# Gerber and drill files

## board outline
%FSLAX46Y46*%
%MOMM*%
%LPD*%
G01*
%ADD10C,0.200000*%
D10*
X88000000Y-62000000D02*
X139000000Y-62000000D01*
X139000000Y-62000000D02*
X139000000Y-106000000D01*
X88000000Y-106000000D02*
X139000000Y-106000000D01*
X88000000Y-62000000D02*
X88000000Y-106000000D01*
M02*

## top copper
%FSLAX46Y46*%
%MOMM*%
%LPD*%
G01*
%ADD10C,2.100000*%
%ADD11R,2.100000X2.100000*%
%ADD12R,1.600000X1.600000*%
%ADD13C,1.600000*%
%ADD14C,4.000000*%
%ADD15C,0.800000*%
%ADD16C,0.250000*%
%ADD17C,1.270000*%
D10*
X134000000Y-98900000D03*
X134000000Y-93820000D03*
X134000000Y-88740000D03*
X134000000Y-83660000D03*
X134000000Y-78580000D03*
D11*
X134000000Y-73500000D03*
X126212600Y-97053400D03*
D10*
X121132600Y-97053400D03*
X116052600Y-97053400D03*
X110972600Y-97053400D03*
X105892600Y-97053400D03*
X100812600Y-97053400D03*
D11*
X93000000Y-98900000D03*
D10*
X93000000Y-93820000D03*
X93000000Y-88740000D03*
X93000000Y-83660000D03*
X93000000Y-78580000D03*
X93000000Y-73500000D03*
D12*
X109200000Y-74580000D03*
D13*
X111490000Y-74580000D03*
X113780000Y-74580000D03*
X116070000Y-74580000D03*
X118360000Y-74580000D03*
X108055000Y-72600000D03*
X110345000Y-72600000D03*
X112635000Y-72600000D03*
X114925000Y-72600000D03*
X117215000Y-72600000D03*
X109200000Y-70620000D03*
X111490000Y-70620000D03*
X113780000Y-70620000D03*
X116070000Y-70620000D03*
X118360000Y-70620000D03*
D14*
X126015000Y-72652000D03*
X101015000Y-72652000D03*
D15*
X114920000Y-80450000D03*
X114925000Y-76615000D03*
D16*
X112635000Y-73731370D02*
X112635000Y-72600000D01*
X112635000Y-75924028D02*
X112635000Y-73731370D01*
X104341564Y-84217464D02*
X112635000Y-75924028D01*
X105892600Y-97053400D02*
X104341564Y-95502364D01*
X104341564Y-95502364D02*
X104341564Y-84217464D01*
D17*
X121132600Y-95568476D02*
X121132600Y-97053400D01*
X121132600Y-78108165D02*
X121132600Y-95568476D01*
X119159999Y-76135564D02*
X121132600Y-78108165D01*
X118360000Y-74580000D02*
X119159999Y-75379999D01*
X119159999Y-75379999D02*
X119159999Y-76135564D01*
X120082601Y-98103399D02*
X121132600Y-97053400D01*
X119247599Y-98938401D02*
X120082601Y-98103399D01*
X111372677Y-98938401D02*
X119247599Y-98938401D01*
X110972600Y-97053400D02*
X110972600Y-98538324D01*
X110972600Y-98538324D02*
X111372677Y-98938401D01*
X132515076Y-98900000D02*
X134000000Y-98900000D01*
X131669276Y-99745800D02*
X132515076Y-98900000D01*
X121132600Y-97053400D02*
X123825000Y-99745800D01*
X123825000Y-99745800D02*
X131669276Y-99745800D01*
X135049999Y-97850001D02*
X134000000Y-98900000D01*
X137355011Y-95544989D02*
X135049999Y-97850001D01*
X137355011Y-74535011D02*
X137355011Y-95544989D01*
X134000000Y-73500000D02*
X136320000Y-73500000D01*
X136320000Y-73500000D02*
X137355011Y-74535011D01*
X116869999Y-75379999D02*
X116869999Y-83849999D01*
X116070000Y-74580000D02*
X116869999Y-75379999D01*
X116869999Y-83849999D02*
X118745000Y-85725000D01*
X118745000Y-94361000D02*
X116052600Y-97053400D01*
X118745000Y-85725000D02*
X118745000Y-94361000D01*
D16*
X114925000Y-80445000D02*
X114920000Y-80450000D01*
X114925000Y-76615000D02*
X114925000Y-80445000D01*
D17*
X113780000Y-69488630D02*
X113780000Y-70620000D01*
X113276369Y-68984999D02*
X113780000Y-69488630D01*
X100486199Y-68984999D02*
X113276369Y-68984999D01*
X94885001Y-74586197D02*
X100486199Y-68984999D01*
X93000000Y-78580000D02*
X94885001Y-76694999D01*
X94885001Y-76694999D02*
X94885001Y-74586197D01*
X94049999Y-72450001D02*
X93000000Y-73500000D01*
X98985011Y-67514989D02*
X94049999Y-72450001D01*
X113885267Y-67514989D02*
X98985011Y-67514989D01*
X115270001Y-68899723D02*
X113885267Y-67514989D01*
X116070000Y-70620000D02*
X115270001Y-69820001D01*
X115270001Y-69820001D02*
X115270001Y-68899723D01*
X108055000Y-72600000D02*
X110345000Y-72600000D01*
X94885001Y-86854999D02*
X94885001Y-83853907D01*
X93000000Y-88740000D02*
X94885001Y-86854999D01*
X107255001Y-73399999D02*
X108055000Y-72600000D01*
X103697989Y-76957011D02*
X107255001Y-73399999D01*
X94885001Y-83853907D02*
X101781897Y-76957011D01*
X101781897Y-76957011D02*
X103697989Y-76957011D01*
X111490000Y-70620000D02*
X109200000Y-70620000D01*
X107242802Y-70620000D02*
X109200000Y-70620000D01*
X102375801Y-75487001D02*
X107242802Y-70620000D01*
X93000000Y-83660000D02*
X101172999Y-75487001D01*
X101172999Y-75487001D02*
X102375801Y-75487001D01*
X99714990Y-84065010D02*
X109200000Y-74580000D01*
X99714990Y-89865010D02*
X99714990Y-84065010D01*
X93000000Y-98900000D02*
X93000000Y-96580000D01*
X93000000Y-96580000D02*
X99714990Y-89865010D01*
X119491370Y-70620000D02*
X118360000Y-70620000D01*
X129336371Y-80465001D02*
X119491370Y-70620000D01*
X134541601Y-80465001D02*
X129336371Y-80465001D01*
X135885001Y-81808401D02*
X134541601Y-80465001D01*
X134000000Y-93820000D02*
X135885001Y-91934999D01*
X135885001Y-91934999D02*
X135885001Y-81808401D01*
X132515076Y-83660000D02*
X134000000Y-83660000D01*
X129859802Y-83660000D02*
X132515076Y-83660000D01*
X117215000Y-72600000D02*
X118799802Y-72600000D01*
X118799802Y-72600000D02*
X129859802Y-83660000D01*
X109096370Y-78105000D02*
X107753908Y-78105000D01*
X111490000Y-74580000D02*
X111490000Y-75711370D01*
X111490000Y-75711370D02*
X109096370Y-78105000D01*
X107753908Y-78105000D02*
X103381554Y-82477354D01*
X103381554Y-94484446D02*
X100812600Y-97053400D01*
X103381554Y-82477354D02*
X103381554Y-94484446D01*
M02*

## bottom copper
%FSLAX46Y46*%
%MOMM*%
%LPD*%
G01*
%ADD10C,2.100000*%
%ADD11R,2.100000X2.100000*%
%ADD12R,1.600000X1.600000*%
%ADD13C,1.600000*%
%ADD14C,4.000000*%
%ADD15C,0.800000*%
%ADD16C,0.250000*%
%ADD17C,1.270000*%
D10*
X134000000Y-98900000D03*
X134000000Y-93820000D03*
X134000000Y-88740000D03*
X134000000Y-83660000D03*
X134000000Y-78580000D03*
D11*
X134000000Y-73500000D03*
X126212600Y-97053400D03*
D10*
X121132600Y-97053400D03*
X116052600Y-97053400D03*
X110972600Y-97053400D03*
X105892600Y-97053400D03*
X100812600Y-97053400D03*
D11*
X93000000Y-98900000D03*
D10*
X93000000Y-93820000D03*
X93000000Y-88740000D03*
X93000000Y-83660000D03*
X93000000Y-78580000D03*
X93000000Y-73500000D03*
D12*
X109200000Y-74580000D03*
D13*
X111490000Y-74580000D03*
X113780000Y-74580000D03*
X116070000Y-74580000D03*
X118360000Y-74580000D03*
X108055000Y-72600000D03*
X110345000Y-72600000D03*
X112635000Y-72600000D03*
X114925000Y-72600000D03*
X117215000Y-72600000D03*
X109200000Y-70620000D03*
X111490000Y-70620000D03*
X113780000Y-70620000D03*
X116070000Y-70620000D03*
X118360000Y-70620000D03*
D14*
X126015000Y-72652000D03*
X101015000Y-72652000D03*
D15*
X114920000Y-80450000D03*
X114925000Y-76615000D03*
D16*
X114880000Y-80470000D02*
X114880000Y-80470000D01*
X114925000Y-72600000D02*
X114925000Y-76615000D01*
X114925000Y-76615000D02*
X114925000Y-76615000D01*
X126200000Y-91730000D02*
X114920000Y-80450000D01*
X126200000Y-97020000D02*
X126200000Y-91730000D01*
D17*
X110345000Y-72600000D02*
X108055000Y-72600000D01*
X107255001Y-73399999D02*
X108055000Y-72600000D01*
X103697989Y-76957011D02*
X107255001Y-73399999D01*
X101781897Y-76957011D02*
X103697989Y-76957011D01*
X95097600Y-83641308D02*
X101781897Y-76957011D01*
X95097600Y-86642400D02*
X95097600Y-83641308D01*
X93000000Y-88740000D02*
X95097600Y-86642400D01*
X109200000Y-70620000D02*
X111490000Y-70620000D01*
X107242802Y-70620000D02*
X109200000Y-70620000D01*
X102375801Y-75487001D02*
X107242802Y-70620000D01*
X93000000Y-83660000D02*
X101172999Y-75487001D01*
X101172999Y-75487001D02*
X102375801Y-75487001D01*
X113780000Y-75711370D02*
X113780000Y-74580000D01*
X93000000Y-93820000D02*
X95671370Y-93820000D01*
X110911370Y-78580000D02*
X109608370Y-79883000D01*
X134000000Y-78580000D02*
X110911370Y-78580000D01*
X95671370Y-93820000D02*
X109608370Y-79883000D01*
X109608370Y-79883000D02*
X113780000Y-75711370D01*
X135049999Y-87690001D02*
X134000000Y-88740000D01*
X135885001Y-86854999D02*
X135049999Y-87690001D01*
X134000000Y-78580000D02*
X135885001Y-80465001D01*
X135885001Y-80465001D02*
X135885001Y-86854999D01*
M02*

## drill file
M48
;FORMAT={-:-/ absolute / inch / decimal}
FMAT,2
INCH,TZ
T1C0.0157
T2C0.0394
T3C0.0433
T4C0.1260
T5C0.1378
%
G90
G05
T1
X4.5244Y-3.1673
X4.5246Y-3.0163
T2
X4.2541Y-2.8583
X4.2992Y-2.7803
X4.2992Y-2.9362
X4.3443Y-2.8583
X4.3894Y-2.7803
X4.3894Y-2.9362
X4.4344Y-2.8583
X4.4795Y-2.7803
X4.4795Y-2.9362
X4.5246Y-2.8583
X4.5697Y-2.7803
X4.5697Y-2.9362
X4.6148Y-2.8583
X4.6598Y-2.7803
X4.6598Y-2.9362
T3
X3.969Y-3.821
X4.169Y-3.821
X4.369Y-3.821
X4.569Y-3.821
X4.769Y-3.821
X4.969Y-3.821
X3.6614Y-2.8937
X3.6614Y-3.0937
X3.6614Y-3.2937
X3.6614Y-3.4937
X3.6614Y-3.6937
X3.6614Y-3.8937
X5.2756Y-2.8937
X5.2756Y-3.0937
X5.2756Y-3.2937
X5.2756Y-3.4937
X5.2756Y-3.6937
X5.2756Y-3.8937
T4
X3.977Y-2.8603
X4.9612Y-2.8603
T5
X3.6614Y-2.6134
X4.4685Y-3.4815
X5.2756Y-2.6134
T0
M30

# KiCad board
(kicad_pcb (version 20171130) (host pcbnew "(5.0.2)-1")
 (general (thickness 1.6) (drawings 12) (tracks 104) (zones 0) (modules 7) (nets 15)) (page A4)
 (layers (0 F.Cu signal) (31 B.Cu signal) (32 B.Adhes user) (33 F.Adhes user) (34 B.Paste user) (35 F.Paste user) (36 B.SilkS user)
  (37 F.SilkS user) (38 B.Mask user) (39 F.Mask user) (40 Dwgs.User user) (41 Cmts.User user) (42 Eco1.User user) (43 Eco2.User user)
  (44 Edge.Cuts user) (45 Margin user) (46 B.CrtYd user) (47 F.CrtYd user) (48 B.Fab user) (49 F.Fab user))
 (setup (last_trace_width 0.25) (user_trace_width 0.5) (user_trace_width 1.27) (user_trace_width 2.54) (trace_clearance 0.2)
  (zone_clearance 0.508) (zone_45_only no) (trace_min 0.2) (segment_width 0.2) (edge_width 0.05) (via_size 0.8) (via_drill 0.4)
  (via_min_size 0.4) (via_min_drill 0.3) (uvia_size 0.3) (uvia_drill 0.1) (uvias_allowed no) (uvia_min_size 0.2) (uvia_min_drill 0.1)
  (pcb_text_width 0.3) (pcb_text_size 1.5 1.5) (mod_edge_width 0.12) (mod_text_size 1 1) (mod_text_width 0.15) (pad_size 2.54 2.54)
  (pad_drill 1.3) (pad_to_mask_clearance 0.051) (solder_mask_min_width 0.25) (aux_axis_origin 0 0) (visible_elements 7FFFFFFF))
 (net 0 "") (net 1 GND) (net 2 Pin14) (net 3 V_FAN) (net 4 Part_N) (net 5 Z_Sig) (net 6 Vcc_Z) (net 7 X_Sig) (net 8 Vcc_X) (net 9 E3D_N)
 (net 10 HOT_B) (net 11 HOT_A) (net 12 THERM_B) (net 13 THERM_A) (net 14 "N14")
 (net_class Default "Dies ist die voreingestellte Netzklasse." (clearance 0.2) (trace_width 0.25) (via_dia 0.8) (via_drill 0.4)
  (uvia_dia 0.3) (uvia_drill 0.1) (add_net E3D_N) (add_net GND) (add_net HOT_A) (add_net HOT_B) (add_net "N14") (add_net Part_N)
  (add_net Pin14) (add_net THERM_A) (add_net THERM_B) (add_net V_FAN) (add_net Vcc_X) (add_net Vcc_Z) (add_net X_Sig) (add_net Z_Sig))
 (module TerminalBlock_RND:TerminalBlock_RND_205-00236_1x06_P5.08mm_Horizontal (layer F.Cu) (at 134 73.5 270)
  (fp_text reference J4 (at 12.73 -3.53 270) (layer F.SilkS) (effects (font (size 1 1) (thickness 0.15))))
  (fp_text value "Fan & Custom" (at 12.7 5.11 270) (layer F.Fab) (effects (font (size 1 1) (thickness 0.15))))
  (pad 6 thru_hole circle (at 25.4 0 270) (size 2.1 2.1) (drill 1.1) (layers *.Cu *.Mask) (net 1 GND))
  (pad 5 thru_hole circle (at 20.32 0 270) (size 2.1 2.1) (drill 1.1) (layers *.Cu *.Mask) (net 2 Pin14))
  (pad 4 thru_hole circle (at 15.24 0 270) (size 2.1 2.1) (drill 1.1) (layers *.Cu *.Mask) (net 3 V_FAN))
  (pad 3 thru_hole circle (at 10.16 0 270) (size 2.1 2.1) (drill 1.1) (layers *.Cu *.Mask) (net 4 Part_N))
  (pad 2 thru_hole circle (at 5.08 0 270) (size 2.1 2.1) (drill 1.1) (layers *.Cu *.Mask) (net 3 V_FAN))
  (pad 1 thru_hole rect (at 0 0 270) (size 2.1 2.1) (drill 1.1) (layers *.Cu *.Mask) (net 1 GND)))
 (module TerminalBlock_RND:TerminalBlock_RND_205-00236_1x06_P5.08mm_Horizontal (layer F.Cu) (at 126.2126 97.0534 180)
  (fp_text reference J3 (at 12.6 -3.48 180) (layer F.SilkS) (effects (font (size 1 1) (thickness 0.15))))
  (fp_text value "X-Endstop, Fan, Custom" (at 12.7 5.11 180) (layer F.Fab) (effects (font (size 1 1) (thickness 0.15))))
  (pad 1 thru_hole rect (at 0 0 180) (size 2.1 2.1) (drill 1.1) (layers *.Cu *.Mask) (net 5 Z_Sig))
  (pad 2 thru_hole circle (at 5.08 0 180) (size 2.1 2.1) (drill 1.1) (layers *.Cu *.Mask) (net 1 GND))
  (pad 3 thru_hole circle (at 10.16 0 180) (size 2.1 2.1) (drill 1.1) (layers *.Cu *.Mask) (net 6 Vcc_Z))
  (pad 4 thru_hole circle (at 15.24 0 180) (size 2.1 2.1) (drill 1.1) (layers *.Cu *.Mask) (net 1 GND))
  (pad 5 thru_hole circle (at 20.32 0 180) (size 2.1 2.1) (drill 1.1) (layers *.Cu *.Mask) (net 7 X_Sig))
  (pad 6 thru_hole circle (at 25.4 0 180) (size 2.1 2.1) (drill 1.1) (layers *.Cu *.Mask) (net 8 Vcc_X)))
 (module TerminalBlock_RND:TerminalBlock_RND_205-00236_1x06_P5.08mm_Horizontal (layer F.Cu) (at 93 98.9 90)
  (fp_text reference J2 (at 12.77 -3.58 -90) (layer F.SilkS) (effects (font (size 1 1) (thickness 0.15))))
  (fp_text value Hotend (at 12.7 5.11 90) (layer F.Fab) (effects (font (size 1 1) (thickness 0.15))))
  (pad 1 thru_hole rect (at 0 0 90) (size 2.1 2.1) (drill 1.1) (layers *.Cu *.Mask) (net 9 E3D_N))
  (pad 2 thru_hole circle (at 5.08 0 90) (size 2.1 2.1) (drill 1.1) (layers *.Cu *.Mask) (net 3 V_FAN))
  (pad 3 thru_hole circle (at 10.16 0 90) (size 2.1 2.1) (drill 1.1) (layers *.Cu *.Mask) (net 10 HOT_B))
  (pad 4 thru_hole circle (at 15.24 0 90) (size 2.1 2.1) (drill 1.1) (layers *.Cu *.Mask) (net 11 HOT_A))
  (pad 5 thru_hole circle (at 20.32 0 90) (size 2.1 2.1) (drill 1.1) (layers *.Cu *.Mask) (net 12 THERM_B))
  (pad 6 thru_hole circle (at 25.4 0 90) (size 2.1 2.1) (drill 1.1) (layers *.Cu *.Mask) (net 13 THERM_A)))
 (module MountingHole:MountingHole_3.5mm (layer F.Cu) (at 113.5 88.43)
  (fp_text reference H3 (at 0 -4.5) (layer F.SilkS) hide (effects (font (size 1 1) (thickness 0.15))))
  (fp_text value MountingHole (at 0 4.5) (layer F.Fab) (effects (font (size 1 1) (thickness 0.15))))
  (pad 1 np_thru_hole circle (at 0 0) (size 3.5 3.5) (drill 3.5) (layers *.Cu *.Mask)))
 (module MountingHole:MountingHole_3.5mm (layer F.Cu) (at 134 66.38)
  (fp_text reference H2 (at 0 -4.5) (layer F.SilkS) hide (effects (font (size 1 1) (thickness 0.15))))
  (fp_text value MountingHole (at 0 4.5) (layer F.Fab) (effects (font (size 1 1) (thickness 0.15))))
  (pad 1 np_thru_hole circle (at 0 0) (size 3.5 3.5) (drill 3.5) (layers *.Cu *.Mask)))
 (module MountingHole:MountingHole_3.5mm (layer F.Cu) (at 93 66.38)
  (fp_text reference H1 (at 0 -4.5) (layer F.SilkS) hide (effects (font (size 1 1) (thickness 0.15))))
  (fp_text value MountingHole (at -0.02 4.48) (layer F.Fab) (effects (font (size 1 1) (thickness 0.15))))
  (pad 1 np_thru_hole circle (at 0 0) (size 3.5 3.5) (drill 3.5) (layers *.Cu *.Mask)))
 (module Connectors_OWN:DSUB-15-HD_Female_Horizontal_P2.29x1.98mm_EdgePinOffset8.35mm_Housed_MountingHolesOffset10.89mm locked (layer F.Cu)
  (at 109.2 74.58 180)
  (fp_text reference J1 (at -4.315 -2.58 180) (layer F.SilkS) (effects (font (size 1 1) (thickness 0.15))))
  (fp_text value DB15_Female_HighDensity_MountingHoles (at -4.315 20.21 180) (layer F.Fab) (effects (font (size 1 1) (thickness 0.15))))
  (pad 1 thru_hole rect (at 0 0 180) (size 1.6 1.6) (drill 1) (layers *.Cu *.Mask) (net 9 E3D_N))
  (pad 2 thru_hole circle (at -2.29 0 180) (size 1.6 1.6) (drill 1) (layers *.Cu *.Mask) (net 8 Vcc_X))
  (pad 3 thru_hole circle (at -4.58 0 180) (size 1.6 1.6) (drill 1) (layers *.Cu *.Mask) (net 3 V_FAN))
  (pad 4 thru_hole circle (at -6.87 0 180) (size 1.6 1.6) (drill 1) (layers *.Cu *.Mask) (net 6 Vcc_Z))
  (pad 5 thru_hole circle (at -9.16 0 180) (size 1.6 1.6) (drill 1) (layers *.Cu *.Mask) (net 1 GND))
  (pad 6 thru_hole circle (at 1.145 1.98 180) (size 1.6 1.6) (drill 1) (layers *.Cu *.Mask) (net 10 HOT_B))
  (pad 7 thru_hole circle (at -1.145 1.98 180) (size 1.6 1.6) (drill 1) (layers *.Cu *.Mask) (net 10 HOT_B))
  (pad 8 thru_hole circle (at -3.435 1.98 180) (size 1.6 1.6) (drill 1) (layers *.Cu *.Mask) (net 7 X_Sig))
  (pad 9 thru_hole circle (at -5.725 1.98 180) (size 1.6 1.6) (drill 1) (layers *.Cu *.Mask) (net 5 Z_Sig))
  (pad 10 thru_hole circle (at -8.015 1.98 180) (size 1.6 1.6) (drill 1) (layers *.Cu *.Mask) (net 4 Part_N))
  (pad 11 thru_hole circle (at 0 3.96 180) (size 1.6 1.6) (drill 1) (layers *.Cu *.Mask) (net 11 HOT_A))
  (pad 12 thru_hole circle (at -2.29 3.96 180) (size 1.6 1.6) (drill 1) (layers *.Cu *.Mask) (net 11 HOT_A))
  (pad 13 thru_hole circle (at -4.58 3.96 180) (size 1.6 1.6) (drill 1) (layers *.Cu *.Mask) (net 12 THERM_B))
  (pad 14 thru_hole circle (at -6.87 3.96 180) (size 1.6 1.6) (drill 1) (layers *.Cu *.Mask) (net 13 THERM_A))
  (pad 15 thru_hole circle (at -9.16 3.96 180) (size 1.6 1.6) (drill 1) (layers *.Cu *.Mask) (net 2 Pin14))
  (pad 0 thru_hole circle (at -16.815 1.928 180) (size 4 4) (drill 3.2) (layers *.Cu *.Mask) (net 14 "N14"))
  (pad 0 thru_hole circle (at 8.185 1.928 180) (size 4 4) (drill 3.2) (layers *.Cu *.Mask) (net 14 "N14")))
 (gr_line (start 88 62) (end 139 62) (layer Edge.Cuts) (width 0.2))
 (gr_line (start 139 62) (end 139 106) (layer Edge.Cuts) (width 0.2))
 (gr_line (start 88 106) (end 139 106) (layer Edge.Cuts) (width 0.2))
 (gr_line (start 88 62) (end 88 106) (layer Edge.Cuts) (width 0.2))
 (segment (start 112.635 73.73137) (end 112.635 72.6) (width 0.25) (layer F.Cu) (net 7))
 (segment (start 112.635 75.924028) (end 112.635 73.73137) (width 0.25) (layer F.Cu) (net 7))
 (segment (start 104.341564 84.217464) (end 112.635 75.924028) (width 0.25) (layer F.Cu) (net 7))
 (segment (start 105.8926 97.0534) (end 104.341564 95.502364) (width 0.25) (layer F.Cu) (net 7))
 (segment (start 104.341564 95.502364) (end 104.341564 84.217464) (width 0.25) (layer F.Cu) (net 7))
 (segment (start 121.1326 95.568476) (end 121.1326 97.0534) (width 1.27) (layer F.Cu) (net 1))
 (segment (start 121.1326 78.108165) (end 121.1326 95.568476) (width 1.27) (layer F.Cu) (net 1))
 (segment (start 119.159999 76.135564) (end 121.1326 78.108165) (width 1.27) (layer F.Cu) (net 1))
 (segment (start 118.36 74.58) (end 119.159999 75.379999) (width 1.27) (layer F.Cu) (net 1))
 (segment (start 119.159999 75.379999) (end 119.159999 76.135564) (width 1.27) (layer F.Cu) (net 1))
 (segment (start 120.082601 98.103399) (end 121.1326 97.0534) (width 1.27) (layer F.Cu) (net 1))
 (segment (start 119.247599 98.938401) (end 120.082601 98.103399) (width 1.27) (layer F.Cu) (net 1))
 (segment (start 111.372677 98.938401) (end 119.247599 98.938401) (width 1.27) (layer F.Cu) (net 1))
 (segment (start 110.9726 97.0534) (end 110.9726 98.538324) (width 1.27) (layer F.Cu) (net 1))
 (segment (start 110.9726 98.538324) (end 111.372677 98.938401) (width 1.27) (layer F.Cu) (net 1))
 (segment (start 132.515076 98.9) (end 134 98.9) (width 1.27) (layer F.Cu) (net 1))
 (segment (start 131.669276 99.7458) (end 132.515076 98.9) (width 1.27) (layer F.Cu) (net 1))
 (segment (start 121.1326 97.0534) (end 123.825 99.7458) (width 1.27) (layer F.Cu) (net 1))
 (segment (start 123.825 99.7458) (end 131.669276 99.7458) (width 1.27) (layer F.Cu) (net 1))
 (segment (start 135.049999 97.850001) (end 134 98.9) (width 1.27) (layer F.Cu) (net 1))
 (segment (start 137.355011 95.544989) (end 135.049999 97.850001) (width 1.27) (layer F.Cu) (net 1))
 (segment (start 137.355011 74.535011) (end 137.355011 95.544989) (width 1.27) (layer F.Cu) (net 1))
 (segment (start 134 73.5) (end 136.32 73.5) (width 1.27) (layer F.Cu) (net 1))
 (segment (start 136.32 73.5) (end 137.355011 74.535011) (width 1.27) (layer F.Cu) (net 1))
 (segment (start 116.869999 75.379999) (end 116.869999 83.849999) (width 1.27) (layer F.Cu) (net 6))
 (segment (start 116.07 74.58) (end 116.869999 75.379999) (width 1.27) (layer F.Cu) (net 6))
 (segment (start 116.869999 83.849999) (end 118.745 85.725) (width 1.27) (layer F.Cu) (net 6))
 (segment (start 118.745 94.361) (end 116.0526 97.0534) (width 1.27) (layer F.Cu) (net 6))
 (segment (start 118.745 85.725) (end 118.745 94.361) (width 1.27) (layer F.Cu) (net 6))
 (segment (start 114.88 80.47) (end 114.88 80.47) (width 0.25) (layer B.Cu) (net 5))
 (via (at 114.92 80.45) (size 0.8) (drill 0.4) (layers F.Cu B.Cu) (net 5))
 (segment (start 114.925 72.6) (end 114.925 76.615) (width 0.25) (layer B.Cu) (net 5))
 (segment (start 114.925 76.615) (end 114.925 76.615) (width 0.25) (layer B.Cu) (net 5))
 (via (at 114.925 76.615) (size 0.8) (drill 0.4) (layers F.Cu B.Cu) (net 5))
 (segment (start 114.925 80.445) (end 114.92 80.45) (width 0.25) (layer F.Cu) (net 5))
 (segment (start 114.925 76.615) (end 114.925 80.445) (width 0.25) (layer F.Cu) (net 5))
 (segment (start 126.2 91.73) (end 114.92 80.45) (width 0.25) (layer B.Cu) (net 5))
 (segment (start 126.2 97.02) (end 126.2 91.73) (width 0.25) (layer B.Cu) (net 5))
 (segment (start 113.78 69.48863) (end 113.78 70.62) (width 1.27) (layer F.Cu) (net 12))
 (segment (start 113.276369 68.984999) (end 113.78 69.48863) (width 1.27) (layer F.Cu) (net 12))
 (segment (start 100.486199 68.984999) (end 113.276369 68.984999) (width 1.27) (layer F.Cu) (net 12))
 (segment (start 94.885001 74.586197) (end 100.486199 68.984999) (width 1.27) (layer F.Cu) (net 12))
 (segment (start 93 78.58) (end 94.885001 76.694999) (width 1.27) (layer F.Cu) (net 12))
 (segment (start 94.885001 76.694999) (end 94.885001 74.586197) (width 1.27) (layer F.Cu) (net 12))
 (segment (start 94.049999 72.450001) (end 93 73.5) (width 1.27) (layer F.Cu) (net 13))
 (segment (start 98.985011 67.514989) (end 94.049999 72.450001) (width 1.27) (layer F.Cu) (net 13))
 (segment (start 113.885267 67.514989) (end 98.985011 67.514989) (width 1.27) (layer F.Cu) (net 13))
 (segment (start 115.270001 68.899723) (end 113.885267 67.514989) (width 1.27) (layer F.Cu) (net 13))
 (segment (start 116.07 70.62) (end 115.270001 69.820001) (width 1.27) (layer F.Cu) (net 13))
 (segment (start 115.270001 69.820001) (end 115.270001 68.899723) (width 1.27) (layer F.Cu) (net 13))
 (segment (start 108.055 72.6) (end 110.345 72.6) (width 1.27) (layer F.Cu) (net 10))
 (segment (start 110.345 72.6) (end 108.055 72.6) (width 1.27) (layer B.Cu) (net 10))
 (segment (start 107.255001 73.399999) (end 108.055 72.6) (width 1.27) (layer B.Cu) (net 10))
 (segment (start 103.697989 76.957011) (end 107.255001 73.399999) (width 1.27) (layer B.Cu) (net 10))
 (segment (start 101.781897 76.957011) (end 103.697989 76.957011) (width 1.27) (layer B.Cu) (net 10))
 (segment (start 95.0976 83.641308) (end 101.781897 76.957011) (width 1.27) (layer B.Cu) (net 10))
 (segment (start 95.0976 86.6424) (end 95.0976 83.641308) (width 1.27) (layer B.Cu) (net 10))
 (segment (start 93 88.74) (end 95.0976 86.6424) (width 1.27) (layer B.Cu) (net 10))
 (segment (start 94.885001 86.854999) (end 94.885001 83.853907) (width 1.27) (layer F.Cu) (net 10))
 (segment (start 93 88.74) (end 94.885001 86.854999) (width 1.27) (layer F.Cu) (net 10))
 (segment (start 107.255001 73.399999) (end 108.055 72.6) (width 1.27) (layer F.Cu) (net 10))
 (segment (start 103.697989 76.957011) (end 107.255001 73.399999) (width 1.27) (layer F.Cu) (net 10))
 (segment (start 94.885001 83.853907) (end 101.781897 76.957011) (width 1.27) (layer F.Cu) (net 10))
 (segment (start 101.781897 76.957011) (end 103.697989 76.957011) (width 1.27) (layer F.Cu) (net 10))
 (segment (start 111.49 70.62) (end 109.2 70.62) (width 1.27) (layer F.Cu) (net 11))
 (segment (start 109.2 70.62) (end 111.49 70.62) (width 1.27) (layer B.Cu) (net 11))
 (segment (start 107.242802 70.62) (end 109.2 70.62) (width 1.27) (layer B.Cu) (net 11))
 (segment (start 102.375801 75.487001) (end 107.242802 70.62) (width 1.27) (layer B.Cu) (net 11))
 (segment (start 93 83.66) (end 101.172999 75.487001) (width 1.27) (layer B.Cu) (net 11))
 (segment (start 101.172999 75.487001) (end 102.375801 75.487001) (width 1.27) (layer B.Cu) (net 11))
 (segment (start 107.242802 70.62) (end 109.2 70.62) (width 1.27) (layer F.Cu) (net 11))
 (segment (start 102.375801 75.487001) (end 107.242802 70.62) (width 1.27) (layer F.Cu) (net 11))
 (segment (start 93 83.66) (end 101.172999 75.487001) (width 1.27) (layer F.Cu) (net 11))
 (segment (start 101.172999 75.487001) (end 102.375801 75.487001) (width 1.27) (layer F.Cu) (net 11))
 (segment (start 99.71499 84.06501) (end 109.2 74.58) (width 1.27) (layer F.Cu) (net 9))
 (segment (start 99.71499 89.86501) (end 99.71499 84.06501) (width 1.27) (layer F.Cu) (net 9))
 (segment (start 93 98.9) (end 93 96.58) (width 1.27) (layer F.Cu) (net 9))
 (segment (start 93 96.58) (end 99.71499 89.86501) (width 1.27) (layer F.Cu) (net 9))
 (segment (start 113.78 75.71137) (end 113.78 74.58) (width 1.27) (layer B.Cu) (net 3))
 (segment (start 93 93.82) (end 95.67137 93.82) (width 1.27) (layer B.Cu) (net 3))
 (segment (start 110.91137 78.58) (end 109.60837 79.883) (width 1.27) (layer B.Cu) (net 3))
 (segment (start 134 78.58) (end 110.91137 78.58) (width 1.27) (layer B.Cu) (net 3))
 (segment (start 95.67137 93.82) (end 109.60837 79.883) (width 1.27) (layer B.Cu) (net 3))
 (segment (start 109.60837 79.883) (end 113.78 75.71137) (width 1.27) (layer B.Cu) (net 3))
 (segment (start 135.049999 87.690001) (end 134 88.74) (width 1.27) (layer B.Cu) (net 3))
 (segment (start 135.885001 86.854999) (end 135.049999 87.690001) (width 1.27) (layer B.Cu) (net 3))
 (segment (start 134 78.58) (end 135.885001 80.465001) (width 1.27) (layer B.Cu) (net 3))
 (segment (start 135.885001 80.465001) (end 135.885001 86.854999) (width 1.27) (layer B.Cu) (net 3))
 (segment (start 119.49137 70.62) (end 118.36 70.62) (width 1.27) (layer F.Cu) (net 2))
 (segment (start 129.336371 80.465001) (end 119.49137 70.62) (width 1.27) (layer F.Cu) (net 2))
 (segment (start 134.541601 80.465001) (end 129.336371 80.465001) (width 1.27) (layer F.Cu) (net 2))
 (segment (start 135.885001 81.808401) (end 134.541601 80.465001) (width 1.27) (layer F.Cu) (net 2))
 (segment (start 134 93.82) (end 135.885001 91.934999) (width 1.27) (layer F.Cu) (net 2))
 (segment (start 135.885001 91.934999) (end 135.885001 81.808401) (width 1.27) (layer F.Cu) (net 2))
 (segment (start 132.515076 83.66) (end 134 83.66) (width 1.27) (layer F.Cu) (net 4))
 (segment (start 129.859802 83.66) (end 132.515076 83.66) (width 1.27) (layer F.Cu) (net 4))
 (segment (start 117.215 72.6) (end 118.799802 72.6) (width 1.27) (layer F.Cu) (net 4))
 (segment (start 118.799802 72.6) (end 129.859802 83.66) (width 1.27) (layer F.Cu) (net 4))
 (segment (start 109.09637 78.105) (end 107.753908 78.105) (width 1.27) (layer F.Cu) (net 8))
 (segment (start 111.49 74.58) (end 111.49 75.71137) (width 1.27) (layer F.Cu) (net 8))
 (segment (start 111.49 75.71137) (end 109.09637 78.105) (width 1.27) (layer F.Cu) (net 8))
 (segment (start 107.753908 78.105) (end 103.381554 82.477354) (width 1.27) (layer F.Cu) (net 8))
 (segment (start 103.381554 94.484446) (end 100.8126 97.0534) (width 1.27) (layer F.Cu) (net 8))
 (segment (start 103.381554 82.477354) (end 103.381554 94.484446) (width 1.27) (layer F.Cu) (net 8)))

